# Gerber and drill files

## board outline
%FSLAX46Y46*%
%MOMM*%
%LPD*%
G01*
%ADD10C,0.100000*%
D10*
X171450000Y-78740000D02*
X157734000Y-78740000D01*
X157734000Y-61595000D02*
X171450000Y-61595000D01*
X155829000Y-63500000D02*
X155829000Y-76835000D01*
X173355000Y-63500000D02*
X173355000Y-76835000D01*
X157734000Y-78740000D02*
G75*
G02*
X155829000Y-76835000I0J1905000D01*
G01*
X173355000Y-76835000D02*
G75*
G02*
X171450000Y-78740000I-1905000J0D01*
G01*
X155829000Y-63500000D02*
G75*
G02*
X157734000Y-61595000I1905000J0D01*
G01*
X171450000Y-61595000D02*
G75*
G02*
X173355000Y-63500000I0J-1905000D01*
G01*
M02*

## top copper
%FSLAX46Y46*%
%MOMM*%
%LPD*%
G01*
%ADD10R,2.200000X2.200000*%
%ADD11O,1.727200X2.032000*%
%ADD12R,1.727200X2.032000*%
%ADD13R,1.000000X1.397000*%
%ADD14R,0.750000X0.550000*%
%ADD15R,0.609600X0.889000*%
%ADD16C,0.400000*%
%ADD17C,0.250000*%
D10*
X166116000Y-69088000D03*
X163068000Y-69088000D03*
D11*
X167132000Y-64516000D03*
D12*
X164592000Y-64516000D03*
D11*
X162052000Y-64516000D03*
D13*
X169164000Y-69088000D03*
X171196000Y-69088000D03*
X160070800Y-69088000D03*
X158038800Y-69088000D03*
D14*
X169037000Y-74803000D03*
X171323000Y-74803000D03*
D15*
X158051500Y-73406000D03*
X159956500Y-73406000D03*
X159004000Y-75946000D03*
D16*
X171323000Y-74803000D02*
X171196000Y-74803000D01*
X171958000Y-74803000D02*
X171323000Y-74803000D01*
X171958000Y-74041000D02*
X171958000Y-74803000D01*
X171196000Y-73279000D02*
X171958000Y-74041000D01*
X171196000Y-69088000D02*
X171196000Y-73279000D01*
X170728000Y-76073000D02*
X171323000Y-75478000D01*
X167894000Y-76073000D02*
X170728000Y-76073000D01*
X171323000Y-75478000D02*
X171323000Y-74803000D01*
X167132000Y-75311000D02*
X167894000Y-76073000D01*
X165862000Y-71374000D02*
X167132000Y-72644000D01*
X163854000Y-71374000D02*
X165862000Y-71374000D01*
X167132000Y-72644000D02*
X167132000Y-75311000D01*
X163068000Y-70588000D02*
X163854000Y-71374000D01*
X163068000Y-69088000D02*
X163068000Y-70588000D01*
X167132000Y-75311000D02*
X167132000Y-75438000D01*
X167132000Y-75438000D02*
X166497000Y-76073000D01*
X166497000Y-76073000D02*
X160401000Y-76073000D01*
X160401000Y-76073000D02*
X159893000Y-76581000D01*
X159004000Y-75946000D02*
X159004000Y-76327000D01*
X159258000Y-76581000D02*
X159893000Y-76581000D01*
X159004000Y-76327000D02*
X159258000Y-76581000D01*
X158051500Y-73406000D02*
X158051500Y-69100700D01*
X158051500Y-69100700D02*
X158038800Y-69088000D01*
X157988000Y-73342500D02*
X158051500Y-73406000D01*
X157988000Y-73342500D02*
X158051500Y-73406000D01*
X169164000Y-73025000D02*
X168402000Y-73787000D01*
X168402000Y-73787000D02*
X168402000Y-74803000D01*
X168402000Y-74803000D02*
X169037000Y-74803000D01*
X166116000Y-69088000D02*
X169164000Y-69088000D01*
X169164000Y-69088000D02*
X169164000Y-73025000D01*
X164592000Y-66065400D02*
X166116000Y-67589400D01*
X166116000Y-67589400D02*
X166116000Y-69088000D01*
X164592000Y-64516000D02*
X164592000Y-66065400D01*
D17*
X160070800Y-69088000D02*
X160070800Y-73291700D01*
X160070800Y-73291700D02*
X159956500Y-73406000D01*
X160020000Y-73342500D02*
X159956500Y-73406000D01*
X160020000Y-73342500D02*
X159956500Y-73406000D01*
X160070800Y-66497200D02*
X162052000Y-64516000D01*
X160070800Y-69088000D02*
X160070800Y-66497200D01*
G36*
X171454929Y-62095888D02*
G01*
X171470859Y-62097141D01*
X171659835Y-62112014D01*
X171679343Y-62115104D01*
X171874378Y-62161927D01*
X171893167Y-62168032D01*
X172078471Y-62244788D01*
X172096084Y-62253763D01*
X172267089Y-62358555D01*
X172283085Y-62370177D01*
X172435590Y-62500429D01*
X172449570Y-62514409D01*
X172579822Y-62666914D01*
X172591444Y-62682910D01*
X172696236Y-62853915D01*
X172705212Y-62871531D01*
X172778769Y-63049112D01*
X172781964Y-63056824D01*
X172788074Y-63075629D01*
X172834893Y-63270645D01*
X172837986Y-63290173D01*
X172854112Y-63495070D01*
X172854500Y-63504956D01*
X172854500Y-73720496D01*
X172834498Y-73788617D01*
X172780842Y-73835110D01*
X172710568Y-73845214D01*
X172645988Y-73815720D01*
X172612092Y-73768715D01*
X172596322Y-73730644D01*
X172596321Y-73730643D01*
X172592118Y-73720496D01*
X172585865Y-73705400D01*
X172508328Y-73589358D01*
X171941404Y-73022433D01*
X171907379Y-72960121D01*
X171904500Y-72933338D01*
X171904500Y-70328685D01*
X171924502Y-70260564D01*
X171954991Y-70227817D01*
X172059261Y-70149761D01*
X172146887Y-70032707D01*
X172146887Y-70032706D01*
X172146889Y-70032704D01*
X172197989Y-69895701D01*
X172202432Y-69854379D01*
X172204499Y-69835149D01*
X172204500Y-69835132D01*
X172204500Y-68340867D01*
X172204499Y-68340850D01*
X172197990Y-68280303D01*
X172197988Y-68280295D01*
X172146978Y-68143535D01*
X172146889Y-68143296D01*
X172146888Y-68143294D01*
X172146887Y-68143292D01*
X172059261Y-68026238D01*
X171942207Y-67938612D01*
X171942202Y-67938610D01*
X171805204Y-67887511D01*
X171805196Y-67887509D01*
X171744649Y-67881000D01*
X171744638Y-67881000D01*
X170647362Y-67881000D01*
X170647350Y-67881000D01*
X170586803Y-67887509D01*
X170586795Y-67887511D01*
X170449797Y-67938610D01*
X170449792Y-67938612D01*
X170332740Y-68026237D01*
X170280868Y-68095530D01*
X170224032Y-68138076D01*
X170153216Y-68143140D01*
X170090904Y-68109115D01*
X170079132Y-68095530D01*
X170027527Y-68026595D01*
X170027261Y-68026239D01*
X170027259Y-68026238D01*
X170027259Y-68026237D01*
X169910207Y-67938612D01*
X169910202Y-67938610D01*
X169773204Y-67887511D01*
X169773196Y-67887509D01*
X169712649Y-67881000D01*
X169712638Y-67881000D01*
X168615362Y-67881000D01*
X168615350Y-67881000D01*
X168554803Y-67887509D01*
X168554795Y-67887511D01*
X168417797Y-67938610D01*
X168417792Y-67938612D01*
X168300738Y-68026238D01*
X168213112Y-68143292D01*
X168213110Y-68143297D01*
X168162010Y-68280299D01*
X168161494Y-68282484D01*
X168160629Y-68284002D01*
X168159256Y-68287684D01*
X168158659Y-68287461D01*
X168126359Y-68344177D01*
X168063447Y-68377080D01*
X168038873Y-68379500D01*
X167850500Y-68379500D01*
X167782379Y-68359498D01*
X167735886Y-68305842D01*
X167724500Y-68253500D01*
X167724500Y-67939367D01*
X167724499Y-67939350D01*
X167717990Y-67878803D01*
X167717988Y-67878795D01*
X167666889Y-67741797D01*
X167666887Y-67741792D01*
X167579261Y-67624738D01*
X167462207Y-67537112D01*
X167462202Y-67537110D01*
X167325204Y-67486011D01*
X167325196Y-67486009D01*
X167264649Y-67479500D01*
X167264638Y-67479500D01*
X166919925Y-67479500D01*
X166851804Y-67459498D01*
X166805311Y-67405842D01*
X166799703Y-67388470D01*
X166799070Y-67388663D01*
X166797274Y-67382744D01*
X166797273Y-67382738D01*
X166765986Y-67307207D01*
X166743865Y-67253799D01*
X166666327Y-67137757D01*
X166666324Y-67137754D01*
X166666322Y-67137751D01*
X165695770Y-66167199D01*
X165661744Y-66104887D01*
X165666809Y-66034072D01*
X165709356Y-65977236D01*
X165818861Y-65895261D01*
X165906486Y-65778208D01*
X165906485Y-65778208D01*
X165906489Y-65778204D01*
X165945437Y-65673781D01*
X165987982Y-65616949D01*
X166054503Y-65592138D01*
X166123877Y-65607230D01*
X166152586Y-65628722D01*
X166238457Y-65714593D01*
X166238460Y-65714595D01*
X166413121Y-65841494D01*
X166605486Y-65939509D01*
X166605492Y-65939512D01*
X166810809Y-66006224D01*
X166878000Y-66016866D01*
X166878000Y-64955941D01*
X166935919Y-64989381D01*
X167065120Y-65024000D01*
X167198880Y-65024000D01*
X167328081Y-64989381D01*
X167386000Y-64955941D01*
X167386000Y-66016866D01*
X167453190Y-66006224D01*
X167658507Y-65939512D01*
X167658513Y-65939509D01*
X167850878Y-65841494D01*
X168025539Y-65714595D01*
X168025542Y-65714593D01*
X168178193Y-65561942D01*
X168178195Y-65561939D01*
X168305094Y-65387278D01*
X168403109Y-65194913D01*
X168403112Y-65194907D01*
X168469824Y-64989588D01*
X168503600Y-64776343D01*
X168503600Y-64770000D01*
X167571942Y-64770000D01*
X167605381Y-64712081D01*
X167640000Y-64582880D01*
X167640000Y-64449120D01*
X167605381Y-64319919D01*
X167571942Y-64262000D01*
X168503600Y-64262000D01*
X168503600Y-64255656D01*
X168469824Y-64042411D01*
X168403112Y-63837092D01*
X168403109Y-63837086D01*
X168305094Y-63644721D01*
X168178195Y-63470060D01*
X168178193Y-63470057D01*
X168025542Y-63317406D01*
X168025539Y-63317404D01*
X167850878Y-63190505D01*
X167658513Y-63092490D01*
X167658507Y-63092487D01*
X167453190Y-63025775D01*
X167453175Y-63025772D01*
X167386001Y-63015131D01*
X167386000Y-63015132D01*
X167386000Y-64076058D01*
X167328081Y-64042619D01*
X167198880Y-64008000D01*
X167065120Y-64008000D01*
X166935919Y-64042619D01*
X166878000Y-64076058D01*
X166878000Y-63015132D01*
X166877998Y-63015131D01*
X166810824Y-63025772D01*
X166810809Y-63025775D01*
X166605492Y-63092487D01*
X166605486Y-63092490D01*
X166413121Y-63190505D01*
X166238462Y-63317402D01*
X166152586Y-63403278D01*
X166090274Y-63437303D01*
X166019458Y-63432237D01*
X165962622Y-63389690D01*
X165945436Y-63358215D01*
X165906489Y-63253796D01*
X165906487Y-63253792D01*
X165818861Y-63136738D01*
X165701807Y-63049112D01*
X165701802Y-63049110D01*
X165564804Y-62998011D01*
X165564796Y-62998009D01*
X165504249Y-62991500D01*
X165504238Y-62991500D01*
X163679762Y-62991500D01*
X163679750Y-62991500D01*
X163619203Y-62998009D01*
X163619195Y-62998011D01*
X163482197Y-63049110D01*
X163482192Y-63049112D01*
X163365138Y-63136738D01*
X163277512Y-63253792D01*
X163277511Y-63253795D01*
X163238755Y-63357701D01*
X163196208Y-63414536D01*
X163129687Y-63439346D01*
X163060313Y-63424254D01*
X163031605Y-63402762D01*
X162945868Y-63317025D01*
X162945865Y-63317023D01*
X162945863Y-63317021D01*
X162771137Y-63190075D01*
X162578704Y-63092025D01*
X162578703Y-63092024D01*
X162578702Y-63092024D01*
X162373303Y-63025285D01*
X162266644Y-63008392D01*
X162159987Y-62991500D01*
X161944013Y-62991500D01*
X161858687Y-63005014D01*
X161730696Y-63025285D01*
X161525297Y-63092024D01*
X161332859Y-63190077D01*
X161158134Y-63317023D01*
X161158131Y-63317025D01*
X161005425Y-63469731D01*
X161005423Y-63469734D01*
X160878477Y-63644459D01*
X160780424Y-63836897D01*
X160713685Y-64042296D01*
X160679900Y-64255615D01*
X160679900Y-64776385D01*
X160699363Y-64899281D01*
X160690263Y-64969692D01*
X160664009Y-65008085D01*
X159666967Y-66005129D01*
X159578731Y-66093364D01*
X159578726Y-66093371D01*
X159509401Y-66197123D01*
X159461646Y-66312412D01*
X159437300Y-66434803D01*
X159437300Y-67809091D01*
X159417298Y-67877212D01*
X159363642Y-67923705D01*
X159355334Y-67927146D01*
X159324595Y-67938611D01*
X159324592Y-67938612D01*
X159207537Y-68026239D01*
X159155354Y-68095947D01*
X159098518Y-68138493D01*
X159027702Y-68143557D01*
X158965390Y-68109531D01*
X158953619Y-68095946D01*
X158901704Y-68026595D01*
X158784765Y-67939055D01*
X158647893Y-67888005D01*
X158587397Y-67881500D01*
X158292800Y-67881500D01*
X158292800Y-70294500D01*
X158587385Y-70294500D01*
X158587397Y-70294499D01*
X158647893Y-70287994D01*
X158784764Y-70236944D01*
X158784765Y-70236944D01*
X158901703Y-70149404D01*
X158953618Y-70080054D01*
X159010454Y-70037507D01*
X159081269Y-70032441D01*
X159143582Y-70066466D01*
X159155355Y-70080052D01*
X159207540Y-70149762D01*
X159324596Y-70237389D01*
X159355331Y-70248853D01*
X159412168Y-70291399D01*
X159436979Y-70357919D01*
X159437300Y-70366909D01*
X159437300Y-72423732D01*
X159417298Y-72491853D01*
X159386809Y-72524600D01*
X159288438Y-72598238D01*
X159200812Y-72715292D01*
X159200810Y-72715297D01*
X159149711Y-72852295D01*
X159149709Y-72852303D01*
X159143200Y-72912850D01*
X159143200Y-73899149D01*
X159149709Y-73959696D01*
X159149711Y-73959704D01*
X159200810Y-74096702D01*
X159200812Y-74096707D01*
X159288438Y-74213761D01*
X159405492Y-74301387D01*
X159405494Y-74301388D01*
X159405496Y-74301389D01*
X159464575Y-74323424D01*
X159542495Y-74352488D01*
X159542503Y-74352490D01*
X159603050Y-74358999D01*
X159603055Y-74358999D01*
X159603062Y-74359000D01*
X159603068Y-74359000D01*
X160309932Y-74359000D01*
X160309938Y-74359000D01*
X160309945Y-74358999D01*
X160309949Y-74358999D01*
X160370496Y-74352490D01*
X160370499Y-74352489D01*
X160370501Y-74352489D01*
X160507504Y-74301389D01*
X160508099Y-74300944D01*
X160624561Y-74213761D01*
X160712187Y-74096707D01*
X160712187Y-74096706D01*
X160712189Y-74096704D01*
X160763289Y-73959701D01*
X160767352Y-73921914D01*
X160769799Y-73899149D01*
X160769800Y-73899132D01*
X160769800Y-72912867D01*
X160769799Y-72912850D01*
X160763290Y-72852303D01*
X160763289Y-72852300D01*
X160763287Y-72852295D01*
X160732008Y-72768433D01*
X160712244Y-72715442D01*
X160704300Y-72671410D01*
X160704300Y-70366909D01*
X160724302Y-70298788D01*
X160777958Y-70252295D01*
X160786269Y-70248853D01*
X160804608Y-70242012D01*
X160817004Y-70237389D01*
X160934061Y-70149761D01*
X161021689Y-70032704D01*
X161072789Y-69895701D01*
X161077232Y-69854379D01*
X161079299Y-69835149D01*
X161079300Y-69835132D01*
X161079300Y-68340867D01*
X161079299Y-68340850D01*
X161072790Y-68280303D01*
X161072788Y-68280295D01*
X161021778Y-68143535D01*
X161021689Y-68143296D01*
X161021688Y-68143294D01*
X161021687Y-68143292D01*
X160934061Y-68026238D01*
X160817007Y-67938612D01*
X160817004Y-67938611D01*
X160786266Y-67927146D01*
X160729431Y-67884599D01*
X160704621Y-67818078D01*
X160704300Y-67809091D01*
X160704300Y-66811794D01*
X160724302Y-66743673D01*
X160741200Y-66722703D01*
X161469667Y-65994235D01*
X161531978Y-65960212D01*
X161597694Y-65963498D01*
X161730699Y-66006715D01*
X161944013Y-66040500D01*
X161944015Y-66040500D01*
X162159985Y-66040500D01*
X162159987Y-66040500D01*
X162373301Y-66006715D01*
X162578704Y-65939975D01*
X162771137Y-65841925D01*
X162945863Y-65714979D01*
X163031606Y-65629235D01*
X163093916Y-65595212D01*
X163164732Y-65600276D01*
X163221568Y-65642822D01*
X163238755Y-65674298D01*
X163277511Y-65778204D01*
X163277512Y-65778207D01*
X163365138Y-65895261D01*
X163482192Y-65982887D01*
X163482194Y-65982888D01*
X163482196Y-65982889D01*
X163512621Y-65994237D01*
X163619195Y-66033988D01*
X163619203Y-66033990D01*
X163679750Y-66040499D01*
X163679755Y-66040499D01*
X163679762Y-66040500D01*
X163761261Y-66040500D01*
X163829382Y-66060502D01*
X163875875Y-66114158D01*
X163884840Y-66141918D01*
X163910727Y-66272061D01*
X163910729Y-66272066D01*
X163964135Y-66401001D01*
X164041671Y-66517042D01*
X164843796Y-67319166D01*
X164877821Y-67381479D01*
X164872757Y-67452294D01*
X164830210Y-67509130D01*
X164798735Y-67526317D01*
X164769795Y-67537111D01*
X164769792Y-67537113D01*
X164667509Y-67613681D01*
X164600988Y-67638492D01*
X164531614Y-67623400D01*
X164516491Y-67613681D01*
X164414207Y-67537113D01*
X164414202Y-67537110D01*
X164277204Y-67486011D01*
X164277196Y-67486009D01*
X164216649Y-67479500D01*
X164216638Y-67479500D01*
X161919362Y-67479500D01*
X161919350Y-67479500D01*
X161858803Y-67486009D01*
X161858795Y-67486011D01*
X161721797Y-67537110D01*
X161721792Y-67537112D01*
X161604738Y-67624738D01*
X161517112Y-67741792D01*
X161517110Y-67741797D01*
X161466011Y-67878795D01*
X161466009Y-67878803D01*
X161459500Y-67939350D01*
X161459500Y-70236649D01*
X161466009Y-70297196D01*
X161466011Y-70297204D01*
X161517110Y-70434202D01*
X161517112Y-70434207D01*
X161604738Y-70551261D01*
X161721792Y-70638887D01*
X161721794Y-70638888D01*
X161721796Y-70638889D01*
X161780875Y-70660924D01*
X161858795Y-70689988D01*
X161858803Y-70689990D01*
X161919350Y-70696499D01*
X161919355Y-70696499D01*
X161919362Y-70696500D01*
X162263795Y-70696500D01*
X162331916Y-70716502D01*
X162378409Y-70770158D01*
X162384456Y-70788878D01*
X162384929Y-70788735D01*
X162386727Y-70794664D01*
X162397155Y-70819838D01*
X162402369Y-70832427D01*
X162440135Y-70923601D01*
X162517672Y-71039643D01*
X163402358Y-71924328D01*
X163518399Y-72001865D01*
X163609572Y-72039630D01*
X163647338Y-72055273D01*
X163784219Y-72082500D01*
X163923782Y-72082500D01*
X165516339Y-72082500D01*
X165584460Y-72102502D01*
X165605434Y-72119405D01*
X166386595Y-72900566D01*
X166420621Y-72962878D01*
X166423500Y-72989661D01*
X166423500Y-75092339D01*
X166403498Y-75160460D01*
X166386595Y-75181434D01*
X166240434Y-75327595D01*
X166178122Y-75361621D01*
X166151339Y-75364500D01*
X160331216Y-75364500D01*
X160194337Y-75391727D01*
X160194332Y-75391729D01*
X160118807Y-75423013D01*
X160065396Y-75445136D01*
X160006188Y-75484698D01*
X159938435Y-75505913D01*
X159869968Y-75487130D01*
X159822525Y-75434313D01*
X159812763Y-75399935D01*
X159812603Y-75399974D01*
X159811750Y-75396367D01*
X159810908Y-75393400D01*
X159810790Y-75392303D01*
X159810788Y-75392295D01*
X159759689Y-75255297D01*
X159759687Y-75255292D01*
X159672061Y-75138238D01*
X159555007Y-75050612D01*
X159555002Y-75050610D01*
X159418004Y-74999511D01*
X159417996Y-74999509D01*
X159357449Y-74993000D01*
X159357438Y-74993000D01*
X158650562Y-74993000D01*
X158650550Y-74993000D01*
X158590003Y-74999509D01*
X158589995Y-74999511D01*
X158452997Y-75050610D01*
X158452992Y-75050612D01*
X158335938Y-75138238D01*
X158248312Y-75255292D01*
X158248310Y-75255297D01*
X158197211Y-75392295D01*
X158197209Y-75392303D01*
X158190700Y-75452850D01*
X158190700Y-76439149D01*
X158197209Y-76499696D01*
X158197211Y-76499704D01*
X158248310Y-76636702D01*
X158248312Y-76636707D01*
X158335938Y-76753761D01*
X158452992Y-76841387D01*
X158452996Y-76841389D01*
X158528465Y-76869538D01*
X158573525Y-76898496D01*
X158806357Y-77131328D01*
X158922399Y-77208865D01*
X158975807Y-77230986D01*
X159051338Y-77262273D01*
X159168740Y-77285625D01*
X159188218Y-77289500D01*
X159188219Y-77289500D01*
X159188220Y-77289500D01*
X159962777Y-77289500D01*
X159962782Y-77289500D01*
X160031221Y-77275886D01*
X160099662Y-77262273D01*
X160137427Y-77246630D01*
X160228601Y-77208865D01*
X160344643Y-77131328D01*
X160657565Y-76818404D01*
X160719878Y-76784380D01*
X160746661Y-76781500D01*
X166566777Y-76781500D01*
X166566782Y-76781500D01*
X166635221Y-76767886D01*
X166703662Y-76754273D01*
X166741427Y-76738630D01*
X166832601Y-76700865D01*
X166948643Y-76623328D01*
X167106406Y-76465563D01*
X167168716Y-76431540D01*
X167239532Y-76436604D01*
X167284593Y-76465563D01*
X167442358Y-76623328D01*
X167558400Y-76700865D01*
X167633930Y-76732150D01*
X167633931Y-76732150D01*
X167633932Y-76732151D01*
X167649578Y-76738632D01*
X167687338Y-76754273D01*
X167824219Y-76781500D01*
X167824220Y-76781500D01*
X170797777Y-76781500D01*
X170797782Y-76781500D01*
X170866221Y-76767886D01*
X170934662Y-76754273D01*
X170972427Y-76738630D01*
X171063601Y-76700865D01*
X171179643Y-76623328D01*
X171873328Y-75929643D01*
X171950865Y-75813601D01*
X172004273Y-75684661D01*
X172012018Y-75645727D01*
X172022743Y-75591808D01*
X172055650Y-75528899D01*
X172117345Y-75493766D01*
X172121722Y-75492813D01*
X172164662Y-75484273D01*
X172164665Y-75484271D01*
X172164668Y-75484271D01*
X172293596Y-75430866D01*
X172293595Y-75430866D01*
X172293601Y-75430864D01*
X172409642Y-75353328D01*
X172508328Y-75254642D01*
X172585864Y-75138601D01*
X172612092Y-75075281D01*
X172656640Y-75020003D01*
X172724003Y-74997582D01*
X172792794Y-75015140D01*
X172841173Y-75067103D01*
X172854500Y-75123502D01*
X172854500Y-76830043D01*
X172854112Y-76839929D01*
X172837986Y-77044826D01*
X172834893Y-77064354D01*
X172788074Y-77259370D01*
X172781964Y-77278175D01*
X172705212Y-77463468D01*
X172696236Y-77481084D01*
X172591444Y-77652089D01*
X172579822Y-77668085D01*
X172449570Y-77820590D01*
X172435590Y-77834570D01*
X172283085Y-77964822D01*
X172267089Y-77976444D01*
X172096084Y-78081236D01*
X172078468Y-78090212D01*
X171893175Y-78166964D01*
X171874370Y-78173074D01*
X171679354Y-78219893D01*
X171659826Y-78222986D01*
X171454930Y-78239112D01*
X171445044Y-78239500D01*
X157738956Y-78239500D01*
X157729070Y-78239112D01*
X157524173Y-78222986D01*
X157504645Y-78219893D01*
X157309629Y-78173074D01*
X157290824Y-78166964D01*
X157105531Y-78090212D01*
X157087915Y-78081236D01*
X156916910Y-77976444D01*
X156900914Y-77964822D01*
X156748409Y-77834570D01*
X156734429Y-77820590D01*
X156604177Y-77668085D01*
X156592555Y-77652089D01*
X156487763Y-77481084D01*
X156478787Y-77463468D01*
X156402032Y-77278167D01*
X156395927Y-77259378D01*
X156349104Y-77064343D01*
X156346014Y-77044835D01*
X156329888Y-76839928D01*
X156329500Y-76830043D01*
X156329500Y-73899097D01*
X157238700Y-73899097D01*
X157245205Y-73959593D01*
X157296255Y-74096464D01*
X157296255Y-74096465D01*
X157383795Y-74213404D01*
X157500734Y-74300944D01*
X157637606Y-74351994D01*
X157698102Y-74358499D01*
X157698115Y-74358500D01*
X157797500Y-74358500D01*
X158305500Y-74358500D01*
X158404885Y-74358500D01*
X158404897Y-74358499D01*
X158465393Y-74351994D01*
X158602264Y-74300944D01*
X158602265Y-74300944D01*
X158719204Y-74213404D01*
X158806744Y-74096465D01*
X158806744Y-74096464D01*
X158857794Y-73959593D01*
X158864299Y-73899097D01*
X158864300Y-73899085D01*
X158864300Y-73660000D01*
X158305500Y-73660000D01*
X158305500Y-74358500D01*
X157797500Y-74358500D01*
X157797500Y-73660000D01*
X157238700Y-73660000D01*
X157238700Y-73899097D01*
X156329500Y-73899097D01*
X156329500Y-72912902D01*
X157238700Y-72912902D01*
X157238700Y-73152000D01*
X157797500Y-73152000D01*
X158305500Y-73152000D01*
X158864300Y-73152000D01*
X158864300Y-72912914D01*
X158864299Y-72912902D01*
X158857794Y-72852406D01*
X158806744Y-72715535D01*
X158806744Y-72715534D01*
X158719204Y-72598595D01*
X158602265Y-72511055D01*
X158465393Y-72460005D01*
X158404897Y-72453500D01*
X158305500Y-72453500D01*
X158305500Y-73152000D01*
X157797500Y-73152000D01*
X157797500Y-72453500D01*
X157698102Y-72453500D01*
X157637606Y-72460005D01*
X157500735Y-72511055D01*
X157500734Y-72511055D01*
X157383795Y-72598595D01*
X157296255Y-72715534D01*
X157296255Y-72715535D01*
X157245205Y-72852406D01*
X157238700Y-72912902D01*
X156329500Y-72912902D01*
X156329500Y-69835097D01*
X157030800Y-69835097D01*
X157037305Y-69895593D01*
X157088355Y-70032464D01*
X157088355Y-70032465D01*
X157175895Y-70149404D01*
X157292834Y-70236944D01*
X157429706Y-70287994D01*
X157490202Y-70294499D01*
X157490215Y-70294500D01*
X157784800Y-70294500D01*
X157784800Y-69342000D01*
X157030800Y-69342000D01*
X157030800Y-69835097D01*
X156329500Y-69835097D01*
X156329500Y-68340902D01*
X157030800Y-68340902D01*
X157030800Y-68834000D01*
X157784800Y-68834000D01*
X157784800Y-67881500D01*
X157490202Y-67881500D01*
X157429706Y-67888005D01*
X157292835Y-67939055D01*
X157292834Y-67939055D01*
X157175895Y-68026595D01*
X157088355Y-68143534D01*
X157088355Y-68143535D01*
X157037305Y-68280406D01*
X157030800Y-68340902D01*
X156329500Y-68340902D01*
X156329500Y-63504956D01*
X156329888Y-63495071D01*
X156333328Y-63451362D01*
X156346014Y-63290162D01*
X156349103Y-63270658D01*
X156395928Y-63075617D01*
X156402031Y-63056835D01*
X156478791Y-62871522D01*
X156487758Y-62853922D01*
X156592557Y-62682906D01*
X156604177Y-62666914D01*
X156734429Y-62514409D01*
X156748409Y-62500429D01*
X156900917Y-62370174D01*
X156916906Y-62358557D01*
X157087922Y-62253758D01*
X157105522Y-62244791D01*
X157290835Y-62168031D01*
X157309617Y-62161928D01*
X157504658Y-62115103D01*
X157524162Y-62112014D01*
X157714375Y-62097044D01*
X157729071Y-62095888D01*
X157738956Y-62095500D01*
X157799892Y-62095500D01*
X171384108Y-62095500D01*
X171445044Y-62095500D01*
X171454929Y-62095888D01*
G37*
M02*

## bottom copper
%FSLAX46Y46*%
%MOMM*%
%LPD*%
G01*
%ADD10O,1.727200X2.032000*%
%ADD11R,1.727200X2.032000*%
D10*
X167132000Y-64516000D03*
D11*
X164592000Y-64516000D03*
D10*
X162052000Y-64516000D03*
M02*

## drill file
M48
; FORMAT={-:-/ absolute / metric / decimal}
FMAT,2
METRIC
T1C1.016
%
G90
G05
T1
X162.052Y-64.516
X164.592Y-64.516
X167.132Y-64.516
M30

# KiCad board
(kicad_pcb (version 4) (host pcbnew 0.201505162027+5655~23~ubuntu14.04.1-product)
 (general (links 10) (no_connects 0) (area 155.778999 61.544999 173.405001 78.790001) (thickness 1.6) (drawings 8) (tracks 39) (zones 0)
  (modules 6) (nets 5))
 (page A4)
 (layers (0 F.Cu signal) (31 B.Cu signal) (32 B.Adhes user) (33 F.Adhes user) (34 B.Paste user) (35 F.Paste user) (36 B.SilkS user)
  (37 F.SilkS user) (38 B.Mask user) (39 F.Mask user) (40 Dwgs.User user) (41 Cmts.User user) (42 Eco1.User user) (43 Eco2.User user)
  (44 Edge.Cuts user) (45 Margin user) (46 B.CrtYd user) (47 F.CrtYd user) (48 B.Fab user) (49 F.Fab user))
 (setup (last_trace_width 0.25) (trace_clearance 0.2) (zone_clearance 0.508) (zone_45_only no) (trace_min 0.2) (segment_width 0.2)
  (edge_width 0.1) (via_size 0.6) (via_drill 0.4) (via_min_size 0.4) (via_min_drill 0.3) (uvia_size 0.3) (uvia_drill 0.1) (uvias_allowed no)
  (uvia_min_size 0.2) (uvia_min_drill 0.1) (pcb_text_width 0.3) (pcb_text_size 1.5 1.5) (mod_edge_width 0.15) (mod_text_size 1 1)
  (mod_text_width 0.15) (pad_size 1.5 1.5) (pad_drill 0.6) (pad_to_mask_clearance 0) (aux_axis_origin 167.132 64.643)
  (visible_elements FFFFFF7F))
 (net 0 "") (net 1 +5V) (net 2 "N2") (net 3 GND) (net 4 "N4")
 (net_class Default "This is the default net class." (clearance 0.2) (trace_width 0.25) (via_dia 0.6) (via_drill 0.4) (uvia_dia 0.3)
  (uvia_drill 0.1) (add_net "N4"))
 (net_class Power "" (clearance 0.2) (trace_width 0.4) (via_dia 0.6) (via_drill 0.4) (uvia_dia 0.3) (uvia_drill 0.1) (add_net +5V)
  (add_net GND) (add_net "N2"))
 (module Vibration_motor (layer F.Cu) (at 164.592 69.088 180)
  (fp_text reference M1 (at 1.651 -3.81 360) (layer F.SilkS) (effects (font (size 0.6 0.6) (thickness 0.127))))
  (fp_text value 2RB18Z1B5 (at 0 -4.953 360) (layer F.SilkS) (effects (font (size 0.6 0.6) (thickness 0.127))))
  (pad 1 smd rect (at -1.524 0 180) (size 2.2 2.2) (layers F.Cu F.Paste F.Mask) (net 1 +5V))
  (pad 2 smd rect (at 1.524 0 180) (size 2.2 2.2) (layers F.Cu F.Paste F.Mask) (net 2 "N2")))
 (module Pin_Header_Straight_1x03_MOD (layer F.Cu) (at 167.132 64.516 270)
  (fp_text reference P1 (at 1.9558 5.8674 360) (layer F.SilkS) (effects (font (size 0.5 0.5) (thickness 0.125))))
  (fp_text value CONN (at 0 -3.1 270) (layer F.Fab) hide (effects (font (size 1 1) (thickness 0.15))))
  (pad 1 thru_hole oval (at 0 0 270) (size 2.032 1.7272) (drill 1.016) (layers *.Cu *.Mask F.SilkS) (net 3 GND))
  (pad 2 thru_hole rect (at 0 2.54 270) (size 2.032 1.7272) (drill 1.016) (layers *.Cu *.Mask F.SilkS) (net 1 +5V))
  (pad 3 thru_hole oval (at 0 5.08 270) (size 2.032 1.7272) (drill 1.016) (layers *.Cu *.Mask F.SilkS) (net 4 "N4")))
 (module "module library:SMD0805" (layer F.Cu) (at 170.18 69.088)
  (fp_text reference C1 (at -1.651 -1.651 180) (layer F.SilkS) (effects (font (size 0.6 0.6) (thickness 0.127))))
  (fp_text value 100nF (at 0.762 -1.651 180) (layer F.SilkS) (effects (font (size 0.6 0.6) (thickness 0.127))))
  (pad 1 smd rect (at -1.016 0) (size 1 1.397) (layers F.Cu F.Paste F.Mask) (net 1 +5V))
  (pad 2 smd rect (at 1.016 0) (size 1 1.397) (layers F.Cu F.Paste F.Mask) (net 2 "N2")))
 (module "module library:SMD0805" (layer F.Cu) (at 159.0548 69.088 180)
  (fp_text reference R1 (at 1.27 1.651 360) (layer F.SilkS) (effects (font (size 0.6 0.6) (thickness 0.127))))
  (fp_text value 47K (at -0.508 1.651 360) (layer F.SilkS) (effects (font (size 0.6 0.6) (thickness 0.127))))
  (pad 1 smd rect (at -1.016 0 180) (size 1 1.397) (layers F.Cu F.Paste F.Mask) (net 4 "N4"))
  (pad 2 smd rect (at 1.016 0 180) (size 1 1.397) (layers F.Cu F.Paste F.Mask) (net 3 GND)))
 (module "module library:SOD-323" (layer F.Cu) (at 170.18 74.803)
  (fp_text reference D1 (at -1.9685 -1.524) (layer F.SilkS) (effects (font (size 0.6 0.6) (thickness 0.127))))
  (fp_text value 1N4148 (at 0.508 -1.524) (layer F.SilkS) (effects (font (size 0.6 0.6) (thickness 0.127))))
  (pad 1 smd rect (at -1.143 0) (size 0.75 0.55) (layers F.Cu F.Paste F.Mask) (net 1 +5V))
  (pad 2 smd rect (at 1.143 0) (size 0.75 0.55) (layers F.Cu F.Paste F.Mask) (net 2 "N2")))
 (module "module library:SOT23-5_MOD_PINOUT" (layer F.Cu) (at 159.004 74.676 180)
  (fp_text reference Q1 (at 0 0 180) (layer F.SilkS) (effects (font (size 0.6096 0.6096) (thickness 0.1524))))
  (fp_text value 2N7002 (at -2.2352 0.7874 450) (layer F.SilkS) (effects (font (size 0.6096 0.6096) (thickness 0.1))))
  (pad 3 smd rect (at 0.9525 1.27 180) (size 0.6096 0.889) (layers F.Cu F.Paste F.Mask) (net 3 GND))
  (pad 2 smd rect (at -0.9525 1.27 180) (size 0.6096 0.889) (layers F.Cu F.Paste F.Mask) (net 4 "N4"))
  (pad 1 smd rect (at 0 -1.27 180) (size 0.6096 0.889) (layers F.Cu F.Paste F.Mask) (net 2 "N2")))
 (gr_line (start 171.45 78.74) (end 157.734 78.74) (angle 90) (layer Edge.Cuts) (width 0.1))
 (gr_line (start 157.734 61.595) (end 171.45 61.595) (angle 90) (layer Edge.Cuts) (width 0.1))
 (gr_line (start 155.829 63.5) (end 155.829 76.835) (angle 90) (layer Edge.Cuts) (width 0.1))
 (gr_line (start 173.355 63.5) (end 173.355 76.835) (angle 90) (layer Edge.Cuts) (width 0.1))
 (gr_arc (start 157.734 76.835) (end 157.734 78.74) (angle 90) (layer Edge.Cuts) (width 0.1))
 (gr_arc (start 171.45 76.835) (end 173.355 76.835) (angle 90) (layer Edge.Cuts) (width 0.1))
 (gr_arc (start 157.734 63.5) (end 155.829 63.5) (angle 90) (layer Edge.Cuts) (width 0.1))
 (gr_arc (start 171.45 63.5) (end 171.45 61.595) (angle 90) (layer Edge.Cuts) (width 0.1))
 (segment (start 171.323 74.803) (end 171.196 74.803) (width 0.4) (layer F.Cu) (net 2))
 (segment (start 171.958 74.803) (end 171.323 74.803) (width 0.4) (layer F.Cu) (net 2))
 (segment (start 171.958 74.041) (end 171.958 74.803) (width 0.4) (layer F.Cu) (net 2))
 (segment (start 171.196 73.279) (end 171.958 74.041) (width 0.4) (layer F.Cu) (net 2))
 (segment (start 171.196 69.088) (end 171.196 73.279) (width 0.4) (layer F.Cu) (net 2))
 (segment (start 170.728 76.073) (end 171.323 75.478) (width 0.4) (layer F.Cu) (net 2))
 (segment (start 167.894 76.073) (end 170.728 76.073) (width 0.4) (layer F.Cu) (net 2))
 (segment (start 171.323 75.478) (end 171.323 74.803) (width 0.4) (layer F.Cu) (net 2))
 (segment (start 167.132 75.311) (end 167.894 76.073) (width 0.4) (layer F.Cu) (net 2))
 (segment (start 165.862 71.374) (end 167.132 72.644) (width 0.4) (layer F.Cu) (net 2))
 (segment (start 163.854 71.374) (end 165.862 71.374) (width 0.4) (layer F.Cu) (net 2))
 (segment (start 167.132 72.644) (end 167.132 75.311) (width 0.4) (layer F.Cu) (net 2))
 (segment (start 163.068 70.588) (end 163.854 71.374) (width 0.4) (layer F.Cu) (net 2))
 (segment (start 163.068 69.088) (end 163.068 70.588) (width 0.4) (layer F.Cu) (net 2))
 (segment (start 167.132 75.311) (end 167.132 75.438) (width 0.4) (layer F.Cu) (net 2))
 (segment (start 167.132 75.438) (end 166.497 76.073) (width 0.4) (layer F.Cu) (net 2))
 (segment (start 166.497 76.073) (end 160.401 76.073) (width 0.4) (layer F.Cu) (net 2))
 (segment (start 160.401 76.073) (end 159.893 76.581) (width 0.4) (layer F.Cu) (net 2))
 (segment (start 159.004 75.946) (end 159.004 76.327) (width 0.4) (layer F.Cu) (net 2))
 (segment (start 159.258 76.581) (end 159.893 76.581) (width 0.4) (layer F.Cu) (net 2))
 (segment (start 159.004 76.327) (end 159.258 76.581) (width 0.4) (layer F.Cu) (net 2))
 (segment (start 158.0515 73.406) (end 158.0515 69.1007) (width 0.4) (layer F.Cu) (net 3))
 (segment (start 158.0515 69.1007) (end 158.0388 69.088) (width 0.4) (layer F.Cu) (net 3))
 (segment (start 157.988 73.3425) (end 158.0515 73.406) (width 0.4) (layer F.Cu) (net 3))
 (segment (start 157.988 73.3425) (end 158.0515 73.406) (width 0.4) (layer F.Cu) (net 3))
 (segment (start 169.164 73.025) (end 168.402 73.787) (width 0.4) (layer F.Cu) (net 1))
 (segment (start 168.402 73.787) (end 168.402 74.803) (width 0.4) (layer F.Cu) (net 1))
 (segment (start 168.402 74.803) (end 169.037 74.803) (width 0.4) (layer F.Cu) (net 1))
 (segment (start 166.116 69.088) (end 169.164 69.088) (width 0.4) (layer F.Cu) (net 1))
 (segment (start 169.164 69.088) (end 169.164 73.025) (width 0.4) (layer F.Cu) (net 1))
 (segment (start 164.592 66.0654) (end 166.116 67.5894) (width 0.4) (layer F.Cu) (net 1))
 (segment (start 166.116 67.5894) (end 166.116 69.088) (width 0.4) (layer F.Cu) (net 1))
 (segment (start 164.592 64.516) (end 164.592 66.0654) (width 0.4) (layer F.Cu) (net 1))
 (segment (start 160.0708 69.088) (end 160.0708 73.2917) (width 0.25) (layer F.Cu) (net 4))
 (segment (start 160.0708 73.2917) (end 159.9565 73.406) (width 0.25) (layer F.Cu) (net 4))
 (segment (start 160.02 73.3425) (end 159.9565 73.406) (width 0.25) (layer F.Cu) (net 4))
 (segment (start 160.02 73.3425) (end 159.9565 73.406) (width 0.25) (layer F.Cu) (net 4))
 (segment (start 160.0708 66.4972) (end 162.052 64.516) (width 0.25) (layer F.Cu) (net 4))
 (segment (start 160.0708 69.088) (end 160.0708 66.4972) (width 0.25) (layer F.Cu) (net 4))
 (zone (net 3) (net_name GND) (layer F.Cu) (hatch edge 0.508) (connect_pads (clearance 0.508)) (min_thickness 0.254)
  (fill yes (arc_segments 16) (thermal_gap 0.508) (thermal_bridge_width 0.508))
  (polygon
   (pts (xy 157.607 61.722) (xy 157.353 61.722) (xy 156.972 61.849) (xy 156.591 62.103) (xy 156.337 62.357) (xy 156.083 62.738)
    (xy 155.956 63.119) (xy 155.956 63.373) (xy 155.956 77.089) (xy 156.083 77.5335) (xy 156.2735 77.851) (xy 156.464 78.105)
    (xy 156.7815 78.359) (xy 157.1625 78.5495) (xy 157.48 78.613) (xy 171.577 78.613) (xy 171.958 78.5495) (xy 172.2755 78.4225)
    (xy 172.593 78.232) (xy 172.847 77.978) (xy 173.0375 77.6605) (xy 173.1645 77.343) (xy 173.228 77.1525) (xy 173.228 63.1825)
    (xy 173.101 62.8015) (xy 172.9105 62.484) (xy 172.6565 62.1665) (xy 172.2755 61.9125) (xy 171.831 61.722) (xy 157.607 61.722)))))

